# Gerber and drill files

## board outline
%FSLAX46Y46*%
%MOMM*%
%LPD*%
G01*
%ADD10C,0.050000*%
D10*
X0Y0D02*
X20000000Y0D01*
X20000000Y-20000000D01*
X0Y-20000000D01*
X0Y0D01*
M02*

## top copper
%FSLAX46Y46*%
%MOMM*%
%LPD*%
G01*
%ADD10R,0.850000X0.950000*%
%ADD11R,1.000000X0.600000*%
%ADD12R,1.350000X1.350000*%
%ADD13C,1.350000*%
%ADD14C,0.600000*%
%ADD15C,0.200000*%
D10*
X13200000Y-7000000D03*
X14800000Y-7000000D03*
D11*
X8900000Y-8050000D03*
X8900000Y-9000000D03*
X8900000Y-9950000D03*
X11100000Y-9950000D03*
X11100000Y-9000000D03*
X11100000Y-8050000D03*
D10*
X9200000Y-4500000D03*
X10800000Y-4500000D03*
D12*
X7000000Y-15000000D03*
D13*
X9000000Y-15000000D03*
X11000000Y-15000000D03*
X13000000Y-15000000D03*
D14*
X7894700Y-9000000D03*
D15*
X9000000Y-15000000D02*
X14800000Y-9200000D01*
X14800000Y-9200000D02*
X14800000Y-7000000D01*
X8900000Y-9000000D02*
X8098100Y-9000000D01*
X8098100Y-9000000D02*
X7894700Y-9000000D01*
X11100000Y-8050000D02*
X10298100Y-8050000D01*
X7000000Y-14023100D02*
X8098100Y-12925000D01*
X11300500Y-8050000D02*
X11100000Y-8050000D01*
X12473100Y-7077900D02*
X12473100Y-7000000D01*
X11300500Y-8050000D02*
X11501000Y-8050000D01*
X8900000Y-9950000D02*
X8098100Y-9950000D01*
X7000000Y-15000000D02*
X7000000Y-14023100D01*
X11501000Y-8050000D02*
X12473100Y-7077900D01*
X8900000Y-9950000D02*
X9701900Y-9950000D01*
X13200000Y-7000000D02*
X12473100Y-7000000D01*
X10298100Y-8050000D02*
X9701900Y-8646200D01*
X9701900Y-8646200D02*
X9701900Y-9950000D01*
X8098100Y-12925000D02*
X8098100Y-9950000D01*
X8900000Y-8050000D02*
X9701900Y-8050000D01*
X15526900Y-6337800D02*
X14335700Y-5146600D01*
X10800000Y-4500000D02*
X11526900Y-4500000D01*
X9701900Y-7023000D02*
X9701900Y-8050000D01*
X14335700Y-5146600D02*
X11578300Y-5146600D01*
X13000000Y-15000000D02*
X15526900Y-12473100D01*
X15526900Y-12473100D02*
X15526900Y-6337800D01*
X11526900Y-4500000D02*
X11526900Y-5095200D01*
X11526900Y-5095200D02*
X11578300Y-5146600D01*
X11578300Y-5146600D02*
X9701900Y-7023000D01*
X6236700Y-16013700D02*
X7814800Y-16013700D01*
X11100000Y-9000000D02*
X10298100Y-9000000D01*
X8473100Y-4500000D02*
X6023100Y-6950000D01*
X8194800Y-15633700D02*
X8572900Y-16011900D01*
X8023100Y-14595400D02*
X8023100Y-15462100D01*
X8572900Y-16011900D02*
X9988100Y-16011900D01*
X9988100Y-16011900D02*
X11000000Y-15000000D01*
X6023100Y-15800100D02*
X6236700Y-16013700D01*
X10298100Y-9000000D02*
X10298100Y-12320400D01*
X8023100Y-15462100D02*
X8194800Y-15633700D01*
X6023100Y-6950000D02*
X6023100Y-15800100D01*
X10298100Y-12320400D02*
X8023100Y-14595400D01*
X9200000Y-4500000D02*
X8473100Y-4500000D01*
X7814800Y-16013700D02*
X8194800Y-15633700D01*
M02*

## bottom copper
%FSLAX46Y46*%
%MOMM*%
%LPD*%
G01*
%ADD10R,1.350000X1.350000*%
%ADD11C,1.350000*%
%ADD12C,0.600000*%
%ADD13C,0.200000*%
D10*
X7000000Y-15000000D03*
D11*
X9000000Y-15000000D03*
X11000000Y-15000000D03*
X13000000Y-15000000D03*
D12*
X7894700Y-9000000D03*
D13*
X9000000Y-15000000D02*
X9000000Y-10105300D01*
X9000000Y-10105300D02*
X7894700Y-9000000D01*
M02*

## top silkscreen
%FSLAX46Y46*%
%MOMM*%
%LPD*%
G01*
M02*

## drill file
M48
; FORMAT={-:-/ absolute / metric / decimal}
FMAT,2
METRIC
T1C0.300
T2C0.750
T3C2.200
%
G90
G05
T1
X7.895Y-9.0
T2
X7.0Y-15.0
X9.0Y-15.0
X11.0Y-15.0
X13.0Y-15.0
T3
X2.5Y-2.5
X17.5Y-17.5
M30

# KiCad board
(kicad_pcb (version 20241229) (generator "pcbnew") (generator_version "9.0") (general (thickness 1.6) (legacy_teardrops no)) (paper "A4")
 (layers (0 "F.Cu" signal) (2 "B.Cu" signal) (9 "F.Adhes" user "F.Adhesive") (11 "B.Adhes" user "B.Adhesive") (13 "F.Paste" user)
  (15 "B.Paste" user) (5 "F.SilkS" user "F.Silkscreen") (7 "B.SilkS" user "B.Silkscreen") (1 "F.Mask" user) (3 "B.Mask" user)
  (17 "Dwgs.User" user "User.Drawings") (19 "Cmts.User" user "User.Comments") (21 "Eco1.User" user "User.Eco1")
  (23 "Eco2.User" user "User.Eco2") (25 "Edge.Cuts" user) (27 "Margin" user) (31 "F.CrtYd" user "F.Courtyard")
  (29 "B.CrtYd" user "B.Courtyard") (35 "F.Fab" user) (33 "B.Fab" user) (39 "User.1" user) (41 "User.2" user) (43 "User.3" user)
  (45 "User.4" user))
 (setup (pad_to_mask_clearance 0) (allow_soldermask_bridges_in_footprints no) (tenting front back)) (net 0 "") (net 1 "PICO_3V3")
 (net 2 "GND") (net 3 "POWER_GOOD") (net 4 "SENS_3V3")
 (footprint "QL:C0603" (layer "F.Cu") (at 14 7)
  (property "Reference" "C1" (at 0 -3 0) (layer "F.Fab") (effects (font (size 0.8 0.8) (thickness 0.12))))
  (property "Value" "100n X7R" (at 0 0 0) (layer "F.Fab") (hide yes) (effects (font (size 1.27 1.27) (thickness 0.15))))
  (pad "1" smd rect (at -0.8 0) (size 0.85 0.95) (layers "F.Cu" "F.Mask" "F.Paste") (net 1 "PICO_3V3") (thermal_bridge_angle 45))
  (pad "2" smd rect (at 0.8 0) (size 0.85 0.95) (layers "F.Cu" "F.Mask" "F.Paste") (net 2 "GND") (thermal_bridge_angle 45)))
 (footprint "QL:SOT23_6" (layer "F.Cu") (at 10 9)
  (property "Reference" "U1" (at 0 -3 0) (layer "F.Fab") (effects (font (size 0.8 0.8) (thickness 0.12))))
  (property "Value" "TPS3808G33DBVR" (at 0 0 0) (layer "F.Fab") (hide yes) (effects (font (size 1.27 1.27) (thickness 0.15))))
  (pad "1" smd rect (at -1.1 -0.95) (size 1 0.6) (layers "F.Cu" "F.Mask" "F.Paste") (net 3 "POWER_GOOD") (thermal_bridge_angle 45))
  (pad "2" smd rect (at -1.1 0) (size 1 0.6) (layers "F.Cu" "F.Mask" "F.Paste") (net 2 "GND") (thermal_bridge_angle 45))
  (pad "3" smd rect (at -1.1 0.95) (size 1 0.6) (layers "F.Cu" "F.Mask" "F.Paste") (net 1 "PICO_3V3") (thermal_bridge_angle 45))
  (pad "4" smd rect (at 1.1 0.95) (size 1 0.6) (layers "F.Cu" "F.Mask" "F.Paste") (thermal_bridge_angle 45))
  (pad "5" smd rect (at 1.1 0) (size 1 0.6) (layers "F.Cu" "F.Mask" "F.Paste") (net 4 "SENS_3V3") (thermal_bridge_angle 45))
  (pad "6" smd rect (at 1.1 -0.95) (size 1 0.6) (layers "F.Cu" "F.Mask" "F.Paste") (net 1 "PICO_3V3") (thermal_bridge_angle 45)))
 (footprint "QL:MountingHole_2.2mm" (layer "F.Cu") (at 2.5 2.5)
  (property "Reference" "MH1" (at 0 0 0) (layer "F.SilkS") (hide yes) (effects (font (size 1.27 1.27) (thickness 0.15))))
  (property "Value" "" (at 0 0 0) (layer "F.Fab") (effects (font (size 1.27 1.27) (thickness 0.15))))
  (pad "" np_thru_hole circle (at 0 0) (size 2.2 2.2) (drill 2.2) (layers "*.Cu" "*.Mask")))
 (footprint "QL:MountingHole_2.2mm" (layer "F.Cu") (at 17.5 17.5)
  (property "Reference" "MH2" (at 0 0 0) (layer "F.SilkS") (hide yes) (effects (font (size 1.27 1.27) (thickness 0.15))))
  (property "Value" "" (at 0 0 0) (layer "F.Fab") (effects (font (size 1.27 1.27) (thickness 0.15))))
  (pad "" np_thru_hole circle (at 0 0) (size 2.2 2.2) (drill 2.2) (layers "*.Cu" "*.Mask")))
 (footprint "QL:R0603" (layer "F.Cu") (at 10 4.5)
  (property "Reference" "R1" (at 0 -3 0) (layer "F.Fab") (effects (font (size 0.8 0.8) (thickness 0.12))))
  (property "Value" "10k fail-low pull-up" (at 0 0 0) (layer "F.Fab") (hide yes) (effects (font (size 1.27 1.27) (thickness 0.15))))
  (pad "1" smd rect (at -0.8 0) (size 0.85 0.95) (layers "F.Cu" "F.Mask" "F.Paste") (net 4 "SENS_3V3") (thermal_bridge_angle 45))
  (pad "2" smd rect (at 0.8 0) (size 0.85 0.95) (layers "F.Cu" "F.Mask" "F.Paste") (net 3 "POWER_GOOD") (thermal_bridge_angle 45)))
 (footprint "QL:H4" (layer "F.Cu") (at 7 15)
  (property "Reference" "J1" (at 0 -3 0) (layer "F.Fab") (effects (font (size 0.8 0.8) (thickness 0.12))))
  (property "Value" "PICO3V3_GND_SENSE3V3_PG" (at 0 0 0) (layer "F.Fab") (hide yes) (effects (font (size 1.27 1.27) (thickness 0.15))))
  (pad "1" thru_hole rect (at 0 0) (size 1.35 1.35) (drill 0.75) (layers "*.Cu" "*.Mask") (remove_unused_layers no) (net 1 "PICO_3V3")
   (thermal_bridge_angle 45))
  (pad "2" thru_hole circle (at 2 0) (size 1.35 1.35) (drill 0.75) (layers "*.Cu" "*.Mask") (remove_unused_layers no) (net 2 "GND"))
  (pad "3" thru_hole circle (at 4 0) (size 1.35 1.35) (drill 0.75) (layers "*.Cu" "*.Mask") (remove_unused_layers no) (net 4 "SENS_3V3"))
  (pad "4" thru_hole circle (at 6 0) (size 1.35 1.35) (drill 0.75) (layers "*.Cu" "*.Mask") (remove_unused_layers no) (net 3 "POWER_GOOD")))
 (gr_rect (start 0 0) (end 20 20) (stroke (width 0.05) (type default)) (fill no) (layer "Edge.Cuts"))
 (segment (start 9 15) (end 14.8 9.2) (width 0.2) (layer "F.Cu") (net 2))
 (segment (start 14.8 9.2) (end 14.8 7) (width 0.2) (layer "F.Cu") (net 2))
 (segment (start 8.9 9) (end 8.0981 9) (width 0.2) (layer "F.Cu") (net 2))
 (segment (start 8.0981 9) (end 7.8947 9) (width 0.2) (layer "F.Cu") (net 2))
 (via (at 7.8947 9) (size 0.6) (drill 0.3) (layers "F.Cu" "B.Cu") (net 2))
 (segment (start 9 15) (end 9 10.1053) (width 0.2) (layer "B.Cu") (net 2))
 (segment (start 9 10.1053) (end 7.8947 9) (width 0.2) (layer "B.Cu") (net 2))
 (segment (start 11.1 8.05) (end 10.2981 8.05) (width 0.2) (layer "F.Cu") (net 1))
 (segment (start 7 14.0231) (end 8.0981 12.925) (width 0.2) (layer "F.Cu") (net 1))
 (segment (start 11.3005 8.05) (end 11.1 8.05) (width 0.2) (layer "F.Cu") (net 1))
 (segment (start 12.4731 7.0779) (end 12.4731 7) (width 0.2) (layer "F.Cu") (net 1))
 (segment (start 11.3005 8.05) (end 11.501 8.05) (width 0.2) (layer "F.Cu") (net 1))
 (segment (start 8.9 9.95) (end 8.0981 9.95) (width 0.2) (layer "F.Cu") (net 1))
 (segment (start 7 15) (end 7 14.0231) (width 0.2) (layer "F.Cu") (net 1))
 (segment (start 11.501 8.05) (end 12.4731 7.0779) (width 0.2) (layer "F.Cu") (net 1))
 (segment (start 8.9 9.95) (end 9.7019 9.95) (width 0.2) (layer "F.Cu") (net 1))
 (segment (start 13.2 7) (end 12.4731 7) (width 0.2) (layer "F.Cu") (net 1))
 (segment (start 10.2981 8.05) (end 9.7019 8.6462) (width 0.2) (layer "F.Cu") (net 1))
 (segment (start 9.7019 8.6462) (end 9.7019 9.95) (width 0.2) (layer "F.Cu") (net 1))
 (segment (start 8.0981 12.925) (end 8.0981 9.95) (width 0.2) (layer "F.Cu") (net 1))
 (segment (start 8.9 8.05) (end 9.7019 8.05) (width 0.2) (layer "F.Cu") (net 3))
 (segment (start 15.5269 6.3378) (end 14.3357 5.1466) (width 0.2) (layer "F.Cu") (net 3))
 (segment (start 10.8 4.5) (end 11.5269 4.5) (width 0.2) (layer "F.Cu") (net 3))
 (segment (start 9.7019 7.023) (end 9.7019 8.05) (width 0.2) (layer "F.Cu") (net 3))
 (segment (start 14.3357 5.1466) (end 11.5783 5.1466) (width 0.2) (layer "F.Cu") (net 3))
 (segment (start 13 15) (end 15.5269 12.4731) (width 0.2) (layer "F.Cu") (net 3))
 (segment (start 15.5269 12.4731) (end 15.5269 6.3378) (width 0.2) (layer "F.Cu") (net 3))
 (segment (start 11.5269 4.5) (end 11.5269 5.0952) (width 0.2) (layer "F.Cu") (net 3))
 (segment (start 11.5269 5.0952) (end 11.5783 5.1466) (width 0.2) (layer "F.Cu") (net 3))
 (segment (start 11.5783 5.1466) (end 9.7019 7.023) (width 0.2) (layer "F.Cu") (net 3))
 (segment (start 6.2367 16.0137) (end 7.8148 16.0137) (width 0.2) (layer "F.Cu") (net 4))
 (segment (start 11.1 9) (end 10.2981 9) (width 0.2) (layer "F.Cu") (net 4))
 (segment (start 8.4731 4.5) (end 6.0231 6.95) (width 0.2) (layer "F.Cu") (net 4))
 (segment (start 8.1948 15.6337) (end 8.5729 16.0119) (width 0.2) (layer "F.Cu") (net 4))
 (segment (start 8.0231 14.5954) (end 8.0231 15.4621) (width 0.2) (layer "F.Cu") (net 4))
 (segment (start 8.5729 16.0119) (end 9.9881 16.0119) (width 0.2) (layer "F.Cu") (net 4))
 (segment (start 9.9881 16.0119) (end 11 15) (width 0.2) (layer "F.Cu") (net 4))
 (segment (start 6.0231 15.8001) (end 6.2367 16.0137) (width 0.2) (layer "F.Cu") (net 4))
 (segment (start 10.2981 9) (end 10.2981 12.3204) (width 0.2) (layer "F.Cu") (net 4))
 (segment (start 8.0231 15.4621) (end 8.1948 15.6337) (width 0.2) (layer "F.Cu") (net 4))
 (segment (start 6.0231 6.95) (end 6.0231 15.8001) (width 0.2) (layer "F.Cu") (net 4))
 (segment (start 10.2981 12.3204) (end 8.0231 14.5954) (width 0.2) (layer "F.Cu") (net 4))
 (segment (start 9.2 4.5) (end 8.4731 4.5) (width 0.2) (layer "F.Cu") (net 4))
 (segment (start 7.8148 16.0137) (end 8.1948 15.6337) (width 0.2) (layer "F.Cu") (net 4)))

